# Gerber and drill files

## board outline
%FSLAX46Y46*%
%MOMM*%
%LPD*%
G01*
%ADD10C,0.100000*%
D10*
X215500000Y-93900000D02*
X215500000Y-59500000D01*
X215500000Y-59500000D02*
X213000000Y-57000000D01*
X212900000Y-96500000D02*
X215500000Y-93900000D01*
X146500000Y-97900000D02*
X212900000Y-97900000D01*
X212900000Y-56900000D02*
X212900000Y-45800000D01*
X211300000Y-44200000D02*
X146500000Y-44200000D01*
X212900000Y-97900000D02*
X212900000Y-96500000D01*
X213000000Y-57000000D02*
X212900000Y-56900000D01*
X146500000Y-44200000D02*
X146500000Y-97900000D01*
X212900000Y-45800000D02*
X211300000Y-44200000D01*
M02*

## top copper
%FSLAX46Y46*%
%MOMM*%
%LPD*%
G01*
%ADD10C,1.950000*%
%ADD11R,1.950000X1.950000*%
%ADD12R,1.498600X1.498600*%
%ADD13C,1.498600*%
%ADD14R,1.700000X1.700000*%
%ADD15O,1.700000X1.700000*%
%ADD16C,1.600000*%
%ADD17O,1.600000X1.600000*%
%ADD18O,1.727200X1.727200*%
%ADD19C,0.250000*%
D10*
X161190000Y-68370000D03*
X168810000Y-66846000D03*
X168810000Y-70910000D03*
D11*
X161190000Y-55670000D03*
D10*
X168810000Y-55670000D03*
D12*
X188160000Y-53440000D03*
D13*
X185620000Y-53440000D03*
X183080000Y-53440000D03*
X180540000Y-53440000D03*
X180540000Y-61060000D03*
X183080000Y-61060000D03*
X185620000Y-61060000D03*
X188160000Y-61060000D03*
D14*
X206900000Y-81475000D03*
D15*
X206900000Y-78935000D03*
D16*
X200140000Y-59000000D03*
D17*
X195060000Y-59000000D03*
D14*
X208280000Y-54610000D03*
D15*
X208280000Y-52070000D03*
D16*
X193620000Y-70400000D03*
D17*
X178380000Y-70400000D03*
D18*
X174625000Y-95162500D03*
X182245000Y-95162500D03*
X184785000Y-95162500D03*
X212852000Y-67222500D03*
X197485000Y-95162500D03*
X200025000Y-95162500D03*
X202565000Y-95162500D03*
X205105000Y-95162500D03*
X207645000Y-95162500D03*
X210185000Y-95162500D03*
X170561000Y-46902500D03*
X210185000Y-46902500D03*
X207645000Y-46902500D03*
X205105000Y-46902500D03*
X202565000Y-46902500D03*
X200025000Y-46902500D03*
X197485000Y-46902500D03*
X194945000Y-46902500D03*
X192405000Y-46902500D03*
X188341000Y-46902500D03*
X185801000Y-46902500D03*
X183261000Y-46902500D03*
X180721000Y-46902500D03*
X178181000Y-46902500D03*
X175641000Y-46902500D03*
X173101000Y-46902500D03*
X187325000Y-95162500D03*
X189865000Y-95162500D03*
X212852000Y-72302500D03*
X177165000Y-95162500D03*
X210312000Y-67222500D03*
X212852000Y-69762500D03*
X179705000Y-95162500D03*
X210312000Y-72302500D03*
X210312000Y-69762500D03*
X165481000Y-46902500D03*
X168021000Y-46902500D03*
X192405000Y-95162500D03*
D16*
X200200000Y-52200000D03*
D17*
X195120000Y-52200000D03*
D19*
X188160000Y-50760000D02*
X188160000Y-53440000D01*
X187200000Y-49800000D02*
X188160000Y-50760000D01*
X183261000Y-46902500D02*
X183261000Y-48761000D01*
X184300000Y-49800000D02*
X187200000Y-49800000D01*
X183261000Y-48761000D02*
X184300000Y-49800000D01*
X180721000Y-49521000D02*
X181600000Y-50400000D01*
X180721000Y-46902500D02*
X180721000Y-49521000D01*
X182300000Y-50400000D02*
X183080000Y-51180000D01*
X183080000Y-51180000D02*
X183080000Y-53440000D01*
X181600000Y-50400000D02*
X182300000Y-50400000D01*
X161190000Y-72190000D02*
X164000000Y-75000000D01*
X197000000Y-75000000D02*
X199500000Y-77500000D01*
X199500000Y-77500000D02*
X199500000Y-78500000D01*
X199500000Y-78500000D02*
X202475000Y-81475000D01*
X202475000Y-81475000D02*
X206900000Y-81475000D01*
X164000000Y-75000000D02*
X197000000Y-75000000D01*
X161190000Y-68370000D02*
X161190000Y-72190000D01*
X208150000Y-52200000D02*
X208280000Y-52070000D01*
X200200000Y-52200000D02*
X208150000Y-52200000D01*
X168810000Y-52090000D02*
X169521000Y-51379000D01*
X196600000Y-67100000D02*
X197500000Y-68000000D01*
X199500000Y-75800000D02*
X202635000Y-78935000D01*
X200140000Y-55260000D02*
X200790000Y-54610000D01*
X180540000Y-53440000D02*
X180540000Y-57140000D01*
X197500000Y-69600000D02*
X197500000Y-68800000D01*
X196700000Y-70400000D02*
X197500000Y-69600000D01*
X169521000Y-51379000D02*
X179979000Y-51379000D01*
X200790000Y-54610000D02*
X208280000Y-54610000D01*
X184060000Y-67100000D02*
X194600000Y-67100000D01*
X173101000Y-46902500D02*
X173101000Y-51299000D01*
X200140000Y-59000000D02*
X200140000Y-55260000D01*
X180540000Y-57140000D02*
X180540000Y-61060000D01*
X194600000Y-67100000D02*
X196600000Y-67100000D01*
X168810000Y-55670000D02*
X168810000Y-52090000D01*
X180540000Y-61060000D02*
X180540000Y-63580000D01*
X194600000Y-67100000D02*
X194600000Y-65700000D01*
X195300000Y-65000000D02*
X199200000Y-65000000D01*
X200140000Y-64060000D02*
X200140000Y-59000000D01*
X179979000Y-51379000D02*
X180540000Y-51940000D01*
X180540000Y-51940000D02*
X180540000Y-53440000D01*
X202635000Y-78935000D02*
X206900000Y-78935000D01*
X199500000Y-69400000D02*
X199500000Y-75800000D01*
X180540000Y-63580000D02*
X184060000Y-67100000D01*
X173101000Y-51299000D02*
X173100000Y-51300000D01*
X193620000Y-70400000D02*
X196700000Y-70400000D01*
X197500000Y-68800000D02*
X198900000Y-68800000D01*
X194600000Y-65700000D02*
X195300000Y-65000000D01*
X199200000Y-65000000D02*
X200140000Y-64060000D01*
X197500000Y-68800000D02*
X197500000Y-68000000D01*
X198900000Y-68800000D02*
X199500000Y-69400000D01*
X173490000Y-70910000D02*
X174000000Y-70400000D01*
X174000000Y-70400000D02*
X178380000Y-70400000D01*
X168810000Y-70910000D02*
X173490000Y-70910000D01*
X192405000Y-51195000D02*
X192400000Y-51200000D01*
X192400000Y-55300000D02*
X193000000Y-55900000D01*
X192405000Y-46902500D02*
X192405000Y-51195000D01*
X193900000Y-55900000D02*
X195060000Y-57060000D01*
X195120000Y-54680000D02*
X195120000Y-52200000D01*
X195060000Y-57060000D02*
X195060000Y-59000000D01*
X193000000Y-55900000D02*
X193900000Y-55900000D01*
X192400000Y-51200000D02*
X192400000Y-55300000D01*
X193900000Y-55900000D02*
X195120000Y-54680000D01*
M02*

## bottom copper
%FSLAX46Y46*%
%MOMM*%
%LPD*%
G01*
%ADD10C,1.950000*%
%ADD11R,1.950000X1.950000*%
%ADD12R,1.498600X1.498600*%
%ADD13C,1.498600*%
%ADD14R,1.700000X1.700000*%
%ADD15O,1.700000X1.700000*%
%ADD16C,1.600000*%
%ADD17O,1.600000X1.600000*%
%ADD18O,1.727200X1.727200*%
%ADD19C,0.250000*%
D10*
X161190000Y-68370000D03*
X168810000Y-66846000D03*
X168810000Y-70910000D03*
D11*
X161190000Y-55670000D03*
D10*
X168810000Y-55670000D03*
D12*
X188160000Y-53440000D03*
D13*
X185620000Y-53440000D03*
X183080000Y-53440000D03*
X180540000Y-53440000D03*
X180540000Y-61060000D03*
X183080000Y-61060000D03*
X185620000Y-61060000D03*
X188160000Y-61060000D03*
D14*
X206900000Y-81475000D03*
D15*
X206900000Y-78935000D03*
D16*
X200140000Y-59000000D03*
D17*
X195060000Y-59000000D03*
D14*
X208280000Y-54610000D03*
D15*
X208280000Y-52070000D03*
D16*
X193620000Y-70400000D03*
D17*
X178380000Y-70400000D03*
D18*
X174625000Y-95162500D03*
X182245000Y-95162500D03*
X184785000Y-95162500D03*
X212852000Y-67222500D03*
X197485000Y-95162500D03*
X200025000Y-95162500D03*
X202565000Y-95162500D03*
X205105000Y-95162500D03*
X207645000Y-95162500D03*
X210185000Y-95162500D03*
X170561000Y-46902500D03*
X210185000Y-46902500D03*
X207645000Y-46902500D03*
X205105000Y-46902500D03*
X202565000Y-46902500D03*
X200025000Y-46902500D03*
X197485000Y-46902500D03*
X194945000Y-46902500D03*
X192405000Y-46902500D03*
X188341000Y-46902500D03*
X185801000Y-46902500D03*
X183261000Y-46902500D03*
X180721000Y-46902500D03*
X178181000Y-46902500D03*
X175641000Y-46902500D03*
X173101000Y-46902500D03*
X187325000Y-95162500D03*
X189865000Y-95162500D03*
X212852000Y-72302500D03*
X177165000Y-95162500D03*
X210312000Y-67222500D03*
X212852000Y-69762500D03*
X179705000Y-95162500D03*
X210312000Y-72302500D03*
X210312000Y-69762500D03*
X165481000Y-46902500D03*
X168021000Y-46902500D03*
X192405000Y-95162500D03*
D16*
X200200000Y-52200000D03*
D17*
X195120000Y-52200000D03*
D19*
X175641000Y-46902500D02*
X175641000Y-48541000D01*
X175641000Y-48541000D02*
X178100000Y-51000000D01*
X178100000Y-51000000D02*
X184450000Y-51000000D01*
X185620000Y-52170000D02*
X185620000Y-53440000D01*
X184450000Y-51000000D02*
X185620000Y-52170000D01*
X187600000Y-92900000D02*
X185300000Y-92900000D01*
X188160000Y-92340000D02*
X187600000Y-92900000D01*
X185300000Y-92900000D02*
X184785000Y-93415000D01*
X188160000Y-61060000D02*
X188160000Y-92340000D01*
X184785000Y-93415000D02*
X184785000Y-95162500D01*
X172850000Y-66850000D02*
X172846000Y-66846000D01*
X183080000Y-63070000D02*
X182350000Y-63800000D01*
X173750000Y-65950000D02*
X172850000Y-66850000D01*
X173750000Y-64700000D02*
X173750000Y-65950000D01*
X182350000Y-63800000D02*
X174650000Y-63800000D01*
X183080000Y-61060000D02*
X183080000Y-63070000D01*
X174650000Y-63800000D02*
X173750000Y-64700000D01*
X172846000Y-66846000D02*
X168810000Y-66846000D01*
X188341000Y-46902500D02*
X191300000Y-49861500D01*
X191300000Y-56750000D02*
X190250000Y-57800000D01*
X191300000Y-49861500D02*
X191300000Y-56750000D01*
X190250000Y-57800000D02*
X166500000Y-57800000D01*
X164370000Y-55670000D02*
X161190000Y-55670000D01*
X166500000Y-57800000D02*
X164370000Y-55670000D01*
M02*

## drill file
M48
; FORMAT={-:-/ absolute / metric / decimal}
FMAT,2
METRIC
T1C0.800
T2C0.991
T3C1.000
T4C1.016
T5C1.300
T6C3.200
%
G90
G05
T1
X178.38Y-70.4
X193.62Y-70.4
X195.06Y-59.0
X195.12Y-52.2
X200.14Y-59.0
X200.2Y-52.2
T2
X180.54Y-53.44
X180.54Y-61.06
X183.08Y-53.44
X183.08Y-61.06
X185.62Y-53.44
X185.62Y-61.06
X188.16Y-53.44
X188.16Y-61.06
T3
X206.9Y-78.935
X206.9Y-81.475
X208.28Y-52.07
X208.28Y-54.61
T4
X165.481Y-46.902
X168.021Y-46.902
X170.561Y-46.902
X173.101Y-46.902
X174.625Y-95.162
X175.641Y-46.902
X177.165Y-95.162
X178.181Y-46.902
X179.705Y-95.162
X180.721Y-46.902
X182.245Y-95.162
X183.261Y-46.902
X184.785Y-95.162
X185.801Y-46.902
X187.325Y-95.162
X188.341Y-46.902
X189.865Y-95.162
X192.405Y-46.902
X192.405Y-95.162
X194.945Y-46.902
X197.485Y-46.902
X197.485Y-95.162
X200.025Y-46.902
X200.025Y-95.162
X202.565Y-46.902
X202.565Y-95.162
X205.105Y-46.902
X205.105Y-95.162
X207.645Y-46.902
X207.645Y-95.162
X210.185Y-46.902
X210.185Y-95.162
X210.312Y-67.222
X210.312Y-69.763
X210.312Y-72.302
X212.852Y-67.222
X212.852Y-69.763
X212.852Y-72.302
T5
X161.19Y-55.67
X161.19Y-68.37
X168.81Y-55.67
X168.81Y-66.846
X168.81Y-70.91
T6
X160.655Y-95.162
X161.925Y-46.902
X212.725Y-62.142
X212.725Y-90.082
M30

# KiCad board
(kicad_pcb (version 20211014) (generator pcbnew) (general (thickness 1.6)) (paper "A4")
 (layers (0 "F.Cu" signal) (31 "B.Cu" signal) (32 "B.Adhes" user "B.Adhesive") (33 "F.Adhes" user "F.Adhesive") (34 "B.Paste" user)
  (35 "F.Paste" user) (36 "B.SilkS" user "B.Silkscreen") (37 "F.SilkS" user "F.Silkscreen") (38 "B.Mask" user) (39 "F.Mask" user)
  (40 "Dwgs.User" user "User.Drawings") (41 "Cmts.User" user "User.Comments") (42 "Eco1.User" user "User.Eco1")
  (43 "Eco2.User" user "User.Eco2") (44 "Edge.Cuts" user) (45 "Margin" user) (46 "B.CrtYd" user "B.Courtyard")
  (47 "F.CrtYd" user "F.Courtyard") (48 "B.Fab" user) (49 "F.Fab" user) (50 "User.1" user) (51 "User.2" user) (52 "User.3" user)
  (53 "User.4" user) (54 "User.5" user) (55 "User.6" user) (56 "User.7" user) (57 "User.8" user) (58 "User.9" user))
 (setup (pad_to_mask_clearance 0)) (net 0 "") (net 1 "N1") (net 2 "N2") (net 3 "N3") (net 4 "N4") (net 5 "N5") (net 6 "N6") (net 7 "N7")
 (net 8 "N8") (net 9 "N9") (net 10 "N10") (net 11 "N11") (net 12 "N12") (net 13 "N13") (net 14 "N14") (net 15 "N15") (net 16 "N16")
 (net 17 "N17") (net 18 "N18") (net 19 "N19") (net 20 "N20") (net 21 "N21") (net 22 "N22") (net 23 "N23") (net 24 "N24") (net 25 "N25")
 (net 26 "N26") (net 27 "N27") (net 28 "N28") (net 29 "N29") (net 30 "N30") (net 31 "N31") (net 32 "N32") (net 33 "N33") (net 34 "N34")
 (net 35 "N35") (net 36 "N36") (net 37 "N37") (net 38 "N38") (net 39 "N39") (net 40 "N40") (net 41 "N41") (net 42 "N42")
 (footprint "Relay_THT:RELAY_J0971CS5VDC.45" (layer "F.Cu") (at 165 63.4 -90)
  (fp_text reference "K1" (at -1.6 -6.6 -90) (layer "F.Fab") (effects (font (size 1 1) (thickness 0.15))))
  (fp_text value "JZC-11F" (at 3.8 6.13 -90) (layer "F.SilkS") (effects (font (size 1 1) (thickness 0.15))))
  (pad "11" thru_hole circle (at 4.97 3.81 270) (size 1.95 1.95) (drill 1.3) (layers *.Cu *.Mask) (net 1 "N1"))
  (pad "12" thru_hole circle (at 3.446 -3.81 270) (size 1.95 1.95) (drill 1.3) (layers *.Cu *.Mask) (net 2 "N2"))
  (pad "14" thru_hole circle (at 7.51 -3.81 270) (size 1.95 1.95) (drill 1.3) (layers *.Cu *.Mask) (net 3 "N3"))
  (pad "A1" thru_hole rect (at -7.73 3.81 270) (size 1.95 1.95) (drill 1.3) (layers *.Cu *.Mask) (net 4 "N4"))
  (pad "A2" thru_hole circle (at -7.73 -3.81 270) (size 1.95 1.95) (drill 1.3) (layers *.Cu *.Mask) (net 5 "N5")))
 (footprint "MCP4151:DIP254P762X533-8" (layer "F.Cu") (at 180.54 61.06 -90)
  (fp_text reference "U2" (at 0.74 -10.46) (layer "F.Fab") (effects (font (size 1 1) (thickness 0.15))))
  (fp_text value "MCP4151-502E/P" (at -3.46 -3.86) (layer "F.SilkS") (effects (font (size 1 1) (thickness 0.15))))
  (pad "1" thru_hole rect locked (at -7.62 -7.62 270) (size 1.4986 1.4986) (drill 0.9906) (layers *.Cu *.Mask) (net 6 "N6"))
  (pad "2" thru_hole circle locked (at -7.62 -5.08 270) (size 1.4986 1.4986) (drill 0.9906) (layers *.Cu *.Mask) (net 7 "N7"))
  (pad "3" thru_hole circle locked (at -7.62 -2.54 270) (size 1.4986 1.4986) (drill 0.9906) (layers *.Cu *.Mask) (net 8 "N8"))
  (pad "4" thru_hole circle locked (at -7.62 0 270) (size 1.4986 1.4986) (drill 0.9906) (layers *.Cu *.Mask) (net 5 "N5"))
  (pad "5" thru_hole circle locked (at 0 0 270) (size 1.4986 1.4986) (drill 0.9906) (layers *.Cu *.Mask) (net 5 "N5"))
  (pad "6" thru_hole circle locked (at 0 -2.54 270) (size 1.4986 1.4986) (drill 0.9906) (layers *.Cu *.Mask) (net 2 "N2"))
  (pad "7" thru_hole circle locked (at 0 -5.08 270) (size 1.4986 1.4986) (drill 0.9906) (layers *.Cu *.Mask) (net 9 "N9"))
  (pad "8" thru_hole circle locked (at 0 -7.62 270) (size 1.4986 1.4986) (drill 0.9906) (layers *.Cu *.Mask) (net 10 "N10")))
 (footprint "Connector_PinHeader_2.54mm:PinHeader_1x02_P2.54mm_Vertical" (layer "F.Cu") (at 206.9 81.475 180)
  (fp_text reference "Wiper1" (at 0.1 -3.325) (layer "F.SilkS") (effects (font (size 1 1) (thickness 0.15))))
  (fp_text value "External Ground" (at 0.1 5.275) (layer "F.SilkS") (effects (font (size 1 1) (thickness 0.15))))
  (pad "1" thru_hole rect (at 0 0 180) (size 1.7 1.7) (drill 1) (layers *.Cu *.Mask) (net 1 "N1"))
  (pad "2" thru_hole oval (at 0 2.54 180) (size 1.7 1.7) (drill 1) (layers *.Cu *.Mask) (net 5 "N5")))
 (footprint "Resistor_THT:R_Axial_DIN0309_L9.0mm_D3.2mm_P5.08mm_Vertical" (layer "F.Cu") (at 200.14 59 180)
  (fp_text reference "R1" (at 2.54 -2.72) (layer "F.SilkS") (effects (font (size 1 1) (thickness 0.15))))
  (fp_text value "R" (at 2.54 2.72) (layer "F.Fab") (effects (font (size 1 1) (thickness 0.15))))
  (pad "1" thru_hole circle (at 0 0 180) (size 1.6 1.6) (drill 0.8) (layers *.Cu *.Mask) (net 5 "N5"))
  (pad "2" thru_hole oval (at 5.08 0 180) (size 1.6 1.6) (drill 0.8) (layers *.Cu *.Mask) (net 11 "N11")))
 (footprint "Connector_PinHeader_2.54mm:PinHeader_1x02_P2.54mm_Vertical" (layer "F.Cu") (at 208.28 54.61 180)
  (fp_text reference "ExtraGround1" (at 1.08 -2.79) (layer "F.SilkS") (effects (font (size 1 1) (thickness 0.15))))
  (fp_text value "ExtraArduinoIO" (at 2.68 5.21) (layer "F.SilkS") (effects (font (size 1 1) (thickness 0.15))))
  (pad "1" thru_hole rect (at 0 0 180) (size 1.7 1.7) (drill 1) (layers *.Cu *.Mask) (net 5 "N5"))
  (pad "2" thru_hole oval (at 0 2.54 180) (size 1.7 1.7) (drill 1) (layers *.Cu *.Mask) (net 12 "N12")))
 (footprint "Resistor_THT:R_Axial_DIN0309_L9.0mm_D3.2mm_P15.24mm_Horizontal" (layer "F.Cu") (at 193.62 70.4 180)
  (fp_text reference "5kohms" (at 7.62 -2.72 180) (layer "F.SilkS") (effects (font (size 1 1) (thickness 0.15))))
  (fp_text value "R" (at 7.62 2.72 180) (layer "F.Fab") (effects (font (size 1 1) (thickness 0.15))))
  (pad "1" thru_hole circle (at 0 0 180) (size 1.6 1.6) (drill 0.8) (layers *.Cu *.Mask) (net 5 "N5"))
  (pad "2" thru_hole oval (at 15.24 0 180) (size 1.6 1.6) (drill 0.8) (layers *.Cu *.Mask) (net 3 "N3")))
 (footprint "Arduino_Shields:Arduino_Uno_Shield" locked (layer "F.Cu") (at 146.685 97.7025)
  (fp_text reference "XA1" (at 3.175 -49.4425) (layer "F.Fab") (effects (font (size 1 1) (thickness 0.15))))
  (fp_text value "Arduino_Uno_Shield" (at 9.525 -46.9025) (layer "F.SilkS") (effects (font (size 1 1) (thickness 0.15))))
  (pad "" np_thru_hole circle locked (at 15.24 -50.8) (size 3.2 3.2) (drill 3.2) (layers *.Cu *.Mask))
  (pad "" np_thru_hole circle locked (at 66.04 -35.56) (size 3.2 3.2) (drill 3.2) (layers *.Cu *.Mask))
  (pad "" np_thru_hole circle locked (at 13.97 -2.54) (size 3.2 3.2) (drill 3.2) (layers *.Cu *.Mask))
  (pad "" np_thru_hole circle locked (at 66.04 -7.62) (size 3.2 3.2) (drill 3.2) (layers *.Cu *.Mask))
  (pad "" thru_hole oval locked (at 27.94 -2.54) (size 1.7272 1.7272) (drill 1.016) (layers *.Cu *.Mask))
  (pad "3V3" thru_hole oval locked (at 35.56 -2.54) (size 1.7272 1.7272) (drill 1.016) (layers *.Cu *.Mask) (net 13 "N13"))
  (pad "5V1" thru_hole oval locked (at 38.1 -2.54) (size 1.7272 1.7272) (drill 1.016) (layers *.Cu *.Mask) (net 10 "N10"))
  (pad "5V2" thru_hole oval locked (at 66.167 -30.48) (size 1.7272 1.7272) (drill 1.016) (layers *.Cu *.Mask) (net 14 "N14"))
  (pad "A0" thru_hole oval locked (at 50.8 -2.54) (size 1.7272 1.7272) (drill 1.016) (layers *.Cu *.Mask) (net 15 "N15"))
  (pad "A1" thru_hole oval locked (at 53.34 -2.54) (size 1.7272 1.7272) (drill 1.016) (layers *.Cu *.Mask) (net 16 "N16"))
  (pad "A2" thru_hole oval locked (at 55.88 -2.54) (size 1.7272 1.7272) (drill 1.016) (layers *.Cu *.Mask) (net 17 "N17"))
  (pad "A3" thru_hole oval locked (at 58.42 -2.54) (size 1.7272 1.7272) (drill 1.016) (layers *.Cu *.Mask) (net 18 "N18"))
  (pad "A4" thru_hole oval locked (at 60.96 -2.54) (size 1.7272 1.7272) (drill 1.016) (layers *.Cu *.Mask) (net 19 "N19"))
  (pad "A5" thru_hole oval locked (at 63.5 -2.54) (size 1.7272 1.7272) (drill 1.016) (layers *.Cu *.Mask) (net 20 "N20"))
  (pad "AREF" thru_hole oval locked (at 23.876 -50.8) (size 1.7272 1.7272) (drill 1.016) (layers *.Cu *.Mask) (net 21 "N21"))
  (pad "D0" thru_hole oval locked (at 63.5 -50.8) (size 1.7272 1.7272) (drill 1.016) (layers *.Cu *.Mask) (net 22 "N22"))
  (pad "D1" thru_hole oval locked (at 60.96 -50.8) (size 1.7272 1.7272) (drill 1.016) (layers *.Cu *.Mask) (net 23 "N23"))
  (pad "D2" thru_hole oval locked (at 58.42 -50.8) (size 1.7272 1.7272) (drill 1.016) (layers *.Cu *.Mask) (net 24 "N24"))
  (pad "D3" thru_hole oval locked (at 55.88 -50.8) (size 1.7272 1.7272) (drill 1.016) (layers *.Cu *.Mask) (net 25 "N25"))
  (pad "D4" thru_hole oval locked (at 53.34 -50.8) (size 1.7272 1.7272) (drill 1.016) (layers *.Cu *.Mask) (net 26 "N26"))
  (pad "D5" thru_hole oval locked (at 50.8 -50.8) (size 1.7272 1.7272) (drill 1.016) (layers *.Cu *.Mask) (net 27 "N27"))
  (pad "D6" thru_hole oval locked (at 48.26 -50.8) (size 1.7272 1.7272) (drill 1.016) (layers *.Cu *.Mask) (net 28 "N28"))
  (pad "D7" thru_hole oval locked (at 45.72 -50.8) (size 1.7272 1.7272) (drill 1.016) (layers *.Cu *.Mask) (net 11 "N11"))
  (pad "D8" thru_hole oval locked (at 41.656 -50.8) (size 1.7272 1.7272) (drill 1.016) (layers *.Cu *.Mask) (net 4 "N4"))
  (pad "D9" thru_hole oval locked (at 39.116 -50.8) (size 1.7272 1.7272) (drill 1.016) (layers *.Cu *.Mask) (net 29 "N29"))
  (pad "D10" thru_hole oval locked (at 36.576 -50.8) (size 1.7272 1.7272) (drill 1.016) (layers *.Cu *.Mask) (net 6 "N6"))
  (pad "D11" thru_hole oval locked (at 34.036 -50.8) (size 1.7272 1.7272) (drill 1.016) (layers *.Cu *.Mask) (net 8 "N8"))
  (pad "D12" thru_hole oval locked (at 31.496 -50.8) (size 1.7272 1.7272) (drill 1.016) (layers *.Cu *.Mask) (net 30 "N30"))
  (pad "D13" thru_hole oval locked (at 28.956 -50.8) (size 1.7272 1.7272) (drill 1.016) (layers *.Cu *.Mask) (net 7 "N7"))
  (pad "GND1" thru_hole oval locked (at 26.416 -50.8) (size 1.7272 1.7272) (drill 1.016) (layers *.Cu *.Mask) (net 5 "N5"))
  (pad "GND2" thru_hole oval locked (at 40.64 -2.54) (size 1.7272 1.7272) (drill 1.016) (layers *.Cu *.Mask) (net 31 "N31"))
  (pad "GND3" thru_hole oval locked (at 43.18 -2.54) (size 1.7272 1.7272) (drill 1.016) (layers *.Cu *.Mask) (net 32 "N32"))
  (pad "GND4" thru_hole oval locked (at 66.167 -25.4) (size 1.7272 1.7272) (drill 1.016) (layers *.Cu *.Mask) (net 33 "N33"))
  (pad "IORF" thru_hole oval locked (at 30.48 -2.54) (size 1.7272 1.7272) (drill 1.016) (layers *.Cu *.Mask) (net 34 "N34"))
  (pad "MISO" thru_hole oval locked (at 63.627 -30.48) (size 1.7272 1.7272) (drill 1.016) (layers *.Cu *.Mask) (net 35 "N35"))
  (pad "MOSI" thru_hole oval locked (at 66.167 -27.94) (size 1.7272 1.7272) (drill 1.016) (layers *.Cu *.Mask) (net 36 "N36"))
  (pad "RST1" thru_hole oval locked (at 33.02 -2.54) (size 1.7272 1.7272) (drill 1.016) (layers *.Cu *.Mask) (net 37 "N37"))
  (pad "RST2" thru_hole oval locked (at 63.627 -25.4) (size 1.7272 1.7272) (drill 1.016) (layers *.Cu *.Mask) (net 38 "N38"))
  (pad "SCK" thru_hole oval locked (at 63.627 -27.94) (size 1.7272 1.7272) (drill 1.016) (layers *.Cu *.Mask) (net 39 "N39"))
  (pad "SCL" thru_hole oval locked (at 18.796 -50.8) (size 1.7272 1.7272) (drill 1.016) (layers *.Cu *.Mask) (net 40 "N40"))
  (pad "SDA" thru_hole oval locked (at 21.336 -50.8) (size 1.7272 1.7272) (drill 1.016) (layers *.Cu *.Mask) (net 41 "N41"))
  (pad "VIN" thru_hole oval locked (at 45.72 -2.54) (size 1.7272 1.7272) (drill 1.016) (layers *.Cu *.Mask) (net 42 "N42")))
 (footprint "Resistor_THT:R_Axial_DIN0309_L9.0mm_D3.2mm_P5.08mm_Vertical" (layer "F.Cu") (at 200.2 52.2 180)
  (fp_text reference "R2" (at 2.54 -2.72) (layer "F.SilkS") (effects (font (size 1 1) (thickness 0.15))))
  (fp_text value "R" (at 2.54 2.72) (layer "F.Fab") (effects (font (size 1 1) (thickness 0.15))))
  (pad "1" thru_hole circle (at 0 0 180) (size 1.6 1.6) (drill 0.8) (layers *.Cu *.Mask) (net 12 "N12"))
  (pad "2" thru_hole oval (at 5.08 0 180) (size 1.6 1.6) (drill 0.8) (layers *.Cu *.Mask) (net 11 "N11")))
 (gr_line (start 215.5 93.9) (end 215.5 59.5) (layer "Edge.Cuts") (width 0.1))
 (gr_line (start 215.5 59.5) (end 213 57) (layer "Edge.Cuts") (width 0.1))
 (gr_line (start 212.9 96.5) (end 215.5 93.9) (layer "Edge.Cuts") (width 0.1))
 (gr_line (start 146.5 97.9) (end 212.9 97.9) (layer "Edge.Cuts") (width 0.1))
 (gr_line (start 212.9 56.9) (end 212.9 45.8) (layer "Edge.Cuts") (width 0.1))
 (gr_line (start 211.3 44.2) (end 146.5 44.2) (layer "Edge.Cuts") (width 0.1))
 (gr_line (start 212.9 97.9) (end 212.9 96.5) (layer "Edge.Cuts") (width 0.1))
 (gr_line (start 213 57) (end 212.9 56.9) (layer "Edge.Cuts") (width 0.1))
 (gr_line (start 146.5 44.2) (end 146.5 97.9) (layer "Edge.Cuts") (width 0.1))
 (gr_line (start 212.9 45.8) (end 211.3 44.2) (layer "Edge.Cuts") (width 0.1))
 (segment (start 188.16 50.76) (end 188.16 53.44) (width 0.25) (layer "F.Cu") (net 6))
 (segment (start 187.2 49.8) (end 188.16 50.76) (width 0.25) (layer "F.Cu") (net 6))
 (segment (start 183.261 46.9025) (end 183.261 48.761) (width 0.25) (layer "F.Cu") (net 6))
 (segment (start 184.3 49.8) (end 187.2 49.8) (width 0.25) (layer "F.Cu") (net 6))
 (segment (start 183.261 48.761) (end 184.3 49.8) (width 0.25) (layer "F.Cu") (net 6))
 (segment (start 175.641 46.9025) (end 175.641 48.541) (width 0.25) (layer "B.Cu") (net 7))
 (segment (start 175.641 48.541) (end 178.1 51) (width 0.25) (layer "B.Cu") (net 7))
 (segment (start 178.1 51) (end 184.45 51) (width 0.25) (layer "B.Cu") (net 7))
 (segment (start 185.62 52.17) (end 185.62 53.44) (width 0.25) (layer "B.Cu") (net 7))
 (segment (start 184.45 51) (end 185.62 52.17) (width 0.25) (layer "B.Cu") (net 7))
 (segment (start 180.721 49.521) (end 181.6 50.4) (width 0.25) (layer "F.Cu") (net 8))
 (segment (start 180.721 46.9025) (end 180.721 49.521) (width 0.25) (layer "F.Cu") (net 8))
 (segment (start 182.3 50.4) (end 183.08 51.18) (width 0.25) (layer "F.Cu") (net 8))
 (segment (start 183.08 51.18) (end 183.08 53.44) (width 0.25) (layer "F.Cu") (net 8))
 (segment (start 181.6 50.4) (end 182.3 50.4) (width 0.25) (layer "F.Cu") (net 8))
 (segment (start 187.6 92.9) (end 185.3 92.9) (width 0.25) (layer "B.Cu") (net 10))
 (segment (start 188.16 92.34) (end 187.6 92.9) (width 0.25) (layer "B.Cu") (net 10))
 (segment (start 185.3 92.9) (end 184.785 93.415) (width 0.25) (layer "B.Cu") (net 10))
 (segment (start 188.16 61.06) (end 188.16 92.34) (width 0.25) (layer "B.Cu") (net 10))
 (segment (start 184.785 93.415) (end 184.785 95.1625) (width 0.25) (layer "B.Cu") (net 10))
 (segment (start 161.19 72.19) (end 164 75) (width 0.25) (layer "F.Cu") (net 1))
 (segment (start 197 75) (end 199.5 77.5) (width 0.25) (layer "F.Cu") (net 1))
 (segment (start 199.5 77.5) (end 199.5 78.5) (width 0.25) (layer "F.Cu") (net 1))
 (segment (start 199.5 78.5) (end 202.475 81.475) (width 0.25) (layer "F.Cu") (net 1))
 (segment (start 202.475 81.475) (end 206.9 81.475) (width 0.25) (layer "F.Cu") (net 1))
 (segment (start 164 75) (end 197 75) (width 0.25) (layer "F.Cu") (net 1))
 (segment (start 161.19 68.37) (end 161.19 72.19) (width 0.25) (layer "F.Cu") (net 1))
 (segment (start 172.85 66.85) (end 172.846 66.846) (width 0.25) (layer "B.Cu") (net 2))
 (segment (start 183.08 63.07) (end 182.35 63.8) (width 0.25) (layer "B.Cu") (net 2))
 (segment (start 173.75 65.95) (end 172.85 66.85) (width 0.25) (layer "B.Cu") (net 2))
 (segment (start 173.75 64.7) (end 173.75 65.95) (width 0.25) (layer "B.Cu") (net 2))
 (segment (start 182.35 63.8) (end 174.65 63.8) (width 0.25) (layer "B.Cu") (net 2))
 (segment (start 183.08 61.06) (end 183.08 63.07) (width 0.25) (layer "B.Cu") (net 2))
 (segment (start 174.65 63.8) (end 173.75 64.7) (width 0.25) (layer "B.Cu") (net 2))
 (segment (start 172.846 66.846) (end 168.81 66.846) (width 0.25) (layer "B.Cu") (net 2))
 (segment (start 188.341 46.9025) (end 191.3 49.8615) (width 0.25) (layer "B.Cu") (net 4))
 (segment (start 191.3 56.75) (end 190.25 57.8) (width 0.25) (layer "B.Cu") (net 4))
 (segment (start 191.3 49.8615) (end 191.3 56.75) (width 0.25) (layer "B.Cu") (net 4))
 (segment (start 190.25 57.8) (end 166.5 57.8) (width 0.25) (layer "B.Cu") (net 4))
 (segment (start 164.37 55.67) (end 161.19 55.67) (width 0.25) (layer "B.Cu") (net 4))
 (segment (start 166.5 57.8) (end 164.37 55.67) (width 0.25) (layer "B.Cu") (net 4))
 (segment (start 208.15 52.2) (end 208.28 52.07) (width 0.25) (layer "F.Cu") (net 12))
 (segment (start 200.2 52.2) (end 208.15 52.2) (width 0.25) (layer "F.Cu") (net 12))
 (segment (start 168.81 52.09) (end 169.521 51.379) (width 0.25) (layer "F.Cu") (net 5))
 (segment (start 196.6 67.1) (end 197.5 68) (width 0.25) (layer "F.Cu") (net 5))
 (segment (start 199.5 75.8) (end 202.635 78.935) (width 0.25) (layer "F.Cu") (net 5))
 (segment (start 200.14 55.26) (end 200.79 54.61) (width 0.25) (layer "F.Cu") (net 5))
 (segment (start 180.54 53.44) (end 180.54 57.14) (width 0.25) (layer "F.Cu") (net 5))
 (segment (start 197.5 69.6) (end 197.5 68.8) (width 0.25) (layer "F.Cu") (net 5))
 (segment (start 196.7 70.4) (end 197.5 69.6) (width 0.25) (layer "F.Cu") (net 5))
 (segment (start 169.521 51.379) (end 179.979 51.379) (width 0.25) (layer "F.Cu") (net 5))
 (segment (start 200.79 54.61) (end 208.28 54.61) (width 0.25) (layer "F.Cu") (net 5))
 (segment (start 184.06 67.1) (end 194.6 67.1) (width 0.25) (layer "F.Cu") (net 5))
 (segment (start 173.101 46.9025) (end 173.101 51.299) (width 0.25) (layer "F.Cu") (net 5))
 (segment (start 200.14 59) (end 200.14 55.26) (width 0.25) (layer "F.Cu") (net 5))
 (segment (start 180.54 57.14) (end 180.54 61.06) (width 0.25) (layer "F.Cu") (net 5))
 (segment (start 194.6 67.1) (end 196.6 67.1) (width 0.25) (layer "F.Cu") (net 5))
 (segment (start 168.81 55.67) (end 168.81 52.09) (width 0.25) (layer "F.Cu") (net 5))
 (segment (start 180.54 61.06) (end 180.54 63.58) (width 0.25) (layer "F.Cu") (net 5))
 (segment (start 194.6 67.1) (end 194.6 65.7) (width 0.25) (layer "F.Cu") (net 5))
 (segment (start 195.3 65) (end 199.2 65) (width 0.25) (layer "F.Cu") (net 5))
 (segment (start 200.14 64.06) (end 200.14 59) (width 0.25) (layer "F.Cu") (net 5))
 (segment (start 179.979 51.379) (end 180.54 51.94) (width 0.25) (layer "F.Cu") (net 5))
 (segment (start 180.54 51.94) (end 180.54 53.44) (width 0.25) (layer "F.Cu") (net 5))
 (segment (start 202.635 78.935) (end 206.9 78.935) (width 0.25) (layer "F.Cu") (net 5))
 (segment (start 199.5 69.4) (end 199.5 75.8) (width 0.25) (layer "F.Cu") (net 5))
 (segment (start 180.54 63.58) (end 184.06 67.1) (width 0.25) (layer "F.Cu") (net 5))
 (segment (start 173.101 51.299) (end 173.1 51.3) (width 0.25) (layer "F.Cu") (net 5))
 (segment (start 193.62 70.4) (end 196.7 70.4) (width 0.25) (layer "F.Cu") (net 5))
 (segment (start 197.5 68.8) (end 198.9 68.8) (width 0.25) (layer "F.Cu") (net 5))
 (segment (start 194.6 65.7) (end 195.3 65) (width 0.25) (layer "F.Cu") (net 5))
 (segment (start 199.2 65) (end 200.14 64.06) (width 0.25) (layer "F.Cu") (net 5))
 (segment (start 197.5 68.8) (end 197.5 68) (width 0.25) (layer "F.Cu") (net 5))
 (segment (start 198.9 68.8) (end 199.5 69.4) (width 0.25) (layer "F.Cu") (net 5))
 (segment (start 173.49 70.91) (end 174 70.4) (width 0.25) (layer "F.Cu") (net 3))
 (segment (start 174 70.4) (end 178.38 70.4) (width 0.25) (layer "F.Cu") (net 3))
 (segment (start 168.81 70.91) (end 173.49 70.91) (width 0.25) (layer "F.Cu") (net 3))
 (segment (start 192.405 51.195) (end 192.4 51.2) (width 0.25) (layer "F.Cu") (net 11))
 (segment (start 192.4 55.3) (end 193 55.9) (width 0.25) (layer "F.Cu") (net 11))
 (segment (start 192.405 46.9025) (end 192.405 51.195) (width 0.25) (layer "F.Cu") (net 11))
 (segment (start 193.9 55.9) (end 195.06 57.06) (width 0.25) (layer "F.Cu") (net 11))
 (segment (start 195.12 54.68) (end 195.12 52.2) (width 0.25) (layer "F.Cu") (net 11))
 (segment (start 195.06 57.06) (end 195.06 59) (width 0.25) (layer "F.Cu") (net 11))
 (segment (start 193 55.9) (end 193.9 55.9) (width 0.25) (layer "F.Cu") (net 11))
 (segment (start 192.4 51.2) (end 192.4 55.3) (width 0.25) (layer "F.Cu") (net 11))
 (segment (start 193.9 55.9) (end 195.12 54.68) (width 0.25) (layer "F.Cu") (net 11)))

